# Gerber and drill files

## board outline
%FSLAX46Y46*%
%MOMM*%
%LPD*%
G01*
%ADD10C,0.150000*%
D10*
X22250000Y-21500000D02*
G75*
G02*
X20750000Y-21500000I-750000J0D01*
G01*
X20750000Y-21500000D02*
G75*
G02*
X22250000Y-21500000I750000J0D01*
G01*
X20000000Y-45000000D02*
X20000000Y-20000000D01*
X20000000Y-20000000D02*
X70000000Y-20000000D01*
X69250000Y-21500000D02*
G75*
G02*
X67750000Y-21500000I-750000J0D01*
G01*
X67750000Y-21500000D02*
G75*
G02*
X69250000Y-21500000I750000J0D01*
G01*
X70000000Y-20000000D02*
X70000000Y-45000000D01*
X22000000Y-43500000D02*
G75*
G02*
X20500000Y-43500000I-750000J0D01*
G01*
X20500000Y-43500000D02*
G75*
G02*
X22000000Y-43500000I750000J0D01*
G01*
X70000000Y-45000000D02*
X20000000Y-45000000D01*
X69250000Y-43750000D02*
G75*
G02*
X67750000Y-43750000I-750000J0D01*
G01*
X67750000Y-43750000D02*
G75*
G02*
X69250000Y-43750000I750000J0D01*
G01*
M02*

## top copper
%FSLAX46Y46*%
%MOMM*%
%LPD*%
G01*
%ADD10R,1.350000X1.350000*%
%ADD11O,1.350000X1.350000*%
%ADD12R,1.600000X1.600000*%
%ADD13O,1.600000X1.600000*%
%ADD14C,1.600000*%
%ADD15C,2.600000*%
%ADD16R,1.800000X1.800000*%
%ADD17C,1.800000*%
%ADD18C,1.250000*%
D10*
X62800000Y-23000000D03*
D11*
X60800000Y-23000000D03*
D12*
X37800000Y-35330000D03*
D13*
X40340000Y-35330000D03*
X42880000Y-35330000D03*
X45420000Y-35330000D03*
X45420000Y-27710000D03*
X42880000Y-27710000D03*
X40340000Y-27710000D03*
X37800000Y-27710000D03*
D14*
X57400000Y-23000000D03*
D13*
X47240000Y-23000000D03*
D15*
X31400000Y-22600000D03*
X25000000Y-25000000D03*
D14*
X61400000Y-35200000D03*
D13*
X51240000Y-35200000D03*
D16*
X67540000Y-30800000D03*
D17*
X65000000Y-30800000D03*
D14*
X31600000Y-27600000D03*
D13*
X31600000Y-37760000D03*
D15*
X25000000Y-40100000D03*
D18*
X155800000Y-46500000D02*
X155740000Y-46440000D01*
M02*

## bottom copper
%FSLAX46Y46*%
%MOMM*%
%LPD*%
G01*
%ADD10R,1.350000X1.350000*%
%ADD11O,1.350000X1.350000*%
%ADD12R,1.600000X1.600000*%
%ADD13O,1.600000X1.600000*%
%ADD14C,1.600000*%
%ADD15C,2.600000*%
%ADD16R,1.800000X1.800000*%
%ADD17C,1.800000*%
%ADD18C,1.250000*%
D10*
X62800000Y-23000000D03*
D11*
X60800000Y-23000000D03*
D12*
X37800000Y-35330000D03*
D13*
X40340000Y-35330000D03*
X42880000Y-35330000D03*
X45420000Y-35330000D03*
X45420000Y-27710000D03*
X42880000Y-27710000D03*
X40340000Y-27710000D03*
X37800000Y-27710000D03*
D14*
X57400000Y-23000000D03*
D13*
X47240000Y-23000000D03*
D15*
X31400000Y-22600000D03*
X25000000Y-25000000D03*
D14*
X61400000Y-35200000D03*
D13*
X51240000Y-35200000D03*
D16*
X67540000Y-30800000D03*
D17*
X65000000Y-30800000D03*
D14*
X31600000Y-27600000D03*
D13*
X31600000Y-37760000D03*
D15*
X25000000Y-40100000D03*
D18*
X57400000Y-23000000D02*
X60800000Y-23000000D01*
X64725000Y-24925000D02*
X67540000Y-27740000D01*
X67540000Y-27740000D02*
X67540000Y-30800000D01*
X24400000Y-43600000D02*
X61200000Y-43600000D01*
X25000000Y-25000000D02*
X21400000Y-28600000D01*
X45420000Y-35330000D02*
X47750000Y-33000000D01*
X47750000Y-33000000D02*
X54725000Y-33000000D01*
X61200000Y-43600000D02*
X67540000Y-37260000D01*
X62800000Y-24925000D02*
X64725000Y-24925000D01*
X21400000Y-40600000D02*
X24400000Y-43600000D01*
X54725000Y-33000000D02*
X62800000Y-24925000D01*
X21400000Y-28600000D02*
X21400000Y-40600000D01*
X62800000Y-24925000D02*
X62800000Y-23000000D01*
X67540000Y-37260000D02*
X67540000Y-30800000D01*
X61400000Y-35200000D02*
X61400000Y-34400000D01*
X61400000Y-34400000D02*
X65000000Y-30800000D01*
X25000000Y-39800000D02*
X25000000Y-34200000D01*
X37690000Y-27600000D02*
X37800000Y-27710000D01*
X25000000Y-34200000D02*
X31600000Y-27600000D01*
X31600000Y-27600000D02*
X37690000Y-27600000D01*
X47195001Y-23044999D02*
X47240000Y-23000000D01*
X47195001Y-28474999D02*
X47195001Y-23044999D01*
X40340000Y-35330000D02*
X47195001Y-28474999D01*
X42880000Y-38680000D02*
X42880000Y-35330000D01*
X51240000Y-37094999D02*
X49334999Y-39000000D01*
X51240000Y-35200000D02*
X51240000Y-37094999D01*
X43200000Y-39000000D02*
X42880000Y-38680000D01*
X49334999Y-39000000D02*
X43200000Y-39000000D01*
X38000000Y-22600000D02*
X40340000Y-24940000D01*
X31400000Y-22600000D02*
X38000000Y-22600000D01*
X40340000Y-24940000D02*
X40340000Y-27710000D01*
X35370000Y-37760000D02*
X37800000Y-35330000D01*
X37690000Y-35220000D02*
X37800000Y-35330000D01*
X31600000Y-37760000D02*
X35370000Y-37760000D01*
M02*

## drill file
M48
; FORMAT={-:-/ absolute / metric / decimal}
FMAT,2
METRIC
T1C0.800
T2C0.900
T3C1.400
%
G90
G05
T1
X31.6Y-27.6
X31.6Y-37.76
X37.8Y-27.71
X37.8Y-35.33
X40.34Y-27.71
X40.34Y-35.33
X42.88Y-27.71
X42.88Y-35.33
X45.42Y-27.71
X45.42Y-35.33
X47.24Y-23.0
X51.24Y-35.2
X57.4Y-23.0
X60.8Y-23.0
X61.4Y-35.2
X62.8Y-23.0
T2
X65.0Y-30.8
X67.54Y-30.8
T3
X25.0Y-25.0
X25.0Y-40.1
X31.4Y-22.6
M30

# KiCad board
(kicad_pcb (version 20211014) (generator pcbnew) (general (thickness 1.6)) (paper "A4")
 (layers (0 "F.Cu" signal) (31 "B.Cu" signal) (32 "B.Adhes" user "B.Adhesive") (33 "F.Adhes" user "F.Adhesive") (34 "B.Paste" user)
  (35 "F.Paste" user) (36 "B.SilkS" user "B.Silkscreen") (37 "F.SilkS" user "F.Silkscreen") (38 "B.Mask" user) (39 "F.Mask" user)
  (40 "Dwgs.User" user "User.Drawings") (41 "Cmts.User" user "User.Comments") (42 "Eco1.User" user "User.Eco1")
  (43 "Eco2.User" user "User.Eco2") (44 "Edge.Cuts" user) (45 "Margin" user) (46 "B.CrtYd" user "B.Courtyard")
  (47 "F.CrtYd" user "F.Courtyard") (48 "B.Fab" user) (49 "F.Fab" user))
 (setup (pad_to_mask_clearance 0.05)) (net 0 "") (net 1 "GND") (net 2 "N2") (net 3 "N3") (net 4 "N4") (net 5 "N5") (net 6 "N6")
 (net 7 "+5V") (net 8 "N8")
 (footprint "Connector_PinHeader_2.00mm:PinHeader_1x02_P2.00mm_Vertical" (layer "F.Cu") (at 62.8 23 -90)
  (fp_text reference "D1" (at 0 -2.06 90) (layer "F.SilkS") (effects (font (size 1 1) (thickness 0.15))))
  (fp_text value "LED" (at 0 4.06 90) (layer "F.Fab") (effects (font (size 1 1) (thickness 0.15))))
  (pad "1" thru_hole rect locked (at 0 0 270) (size 1.35 1.35) (drill 0.8) (layers *.Cu *.Mask) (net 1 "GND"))
  (pad "2" thru_hole oval locked (at 0 2 270) (size 1.35 1.35) (drill 0.8) (layers *.Cu *.Mask) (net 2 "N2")))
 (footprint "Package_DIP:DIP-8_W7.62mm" (layer "F.Cu") (at 37.8 35.33 90)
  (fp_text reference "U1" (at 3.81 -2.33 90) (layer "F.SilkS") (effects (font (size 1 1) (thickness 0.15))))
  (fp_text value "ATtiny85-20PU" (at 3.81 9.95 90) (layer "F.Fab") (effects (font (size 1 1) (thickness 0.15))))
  (pad "1" thru_hole rect locked (at 0 0 90) (size 1.6 1.6) (drill 0.8) (layers *.Cu *.Mask) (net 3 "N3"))
  (pad "2" thru_hole oval locked (at 0 2.54 90) (size 1.6 1.6) (drill 0.8) (layers *.Cu *.Mask) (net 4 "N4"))
  (pad "3" thru_hole oval locked (at 0 5.08 90) (size 1.6 1.6) (drill 0.8) (layers *.Cu *.Mask) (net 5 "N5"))
  (pad "4" thru_hole oval locked (at 0 7.62 90) (size 1.6 1.6) (drill 0.8) (layers *.Cu *.Mask) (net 1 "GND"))
  (pad "5" thru_hole oval locked (at 7.62 7.62 90) (size 1.6 1.6) (drill 0.8) (layers *.Cu *.Mask))
  (pad "6" thru_hole oval locked (at 7.62 5.08 90) (size 1.6 1.6) (drill 0.8) (layers *.Cu *.Mask))
  (pad "7" thru_hole oval locked (at 7.62 2.54 90) (size 1.6 1.6) (drill 0.8) (layers *.Cu *.Mask) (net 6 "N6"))
  (pad "8" thru_hole oval locked (at 7.62 0 90) (size 1.6 1.6) (drill 0.8) (layers *.Cu *.Mask) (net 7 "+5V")))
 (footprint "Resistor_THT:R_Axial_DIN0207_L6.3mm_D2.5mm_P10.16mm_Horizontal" (layer "F.Cu") (at 57.4 23 180)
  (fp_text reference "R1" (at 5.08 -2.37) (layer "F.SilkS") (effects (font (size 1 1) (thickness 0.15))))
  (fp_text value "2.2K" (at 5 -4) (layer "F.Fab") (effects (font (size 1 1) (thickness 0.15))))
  (pad "1" thru_hole circle locked (at 0 0 180) (size 1.6 1.6) (drill 0.8) (layers *.Cu *.Mask) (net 2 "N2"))
  (pad "2" thru_hole oval locked (at 10.16 0 180) (size 1.6 1.6) (drill 0.8) (layers *.Cu *.Mask) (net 4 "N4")))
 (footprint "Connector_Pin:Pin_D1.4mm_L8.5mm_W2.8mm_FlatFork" (layer "F.Cu") (at 31.4 22.6)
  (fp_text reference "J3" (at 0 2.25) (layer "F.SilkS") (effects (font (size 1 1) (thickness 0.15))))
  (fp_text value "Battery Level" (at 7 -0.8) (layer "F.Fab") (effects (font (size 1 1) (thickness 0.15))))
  (pad "1" thru_hole circle locked (at 0 0) (size 2.6 2.6) (drill 1.4) (layers *.Cu *.Mask) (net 6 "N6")))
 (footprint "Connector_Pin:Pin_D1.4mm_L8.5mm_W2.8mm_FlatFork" (layer "F.Cu") (at 25 25)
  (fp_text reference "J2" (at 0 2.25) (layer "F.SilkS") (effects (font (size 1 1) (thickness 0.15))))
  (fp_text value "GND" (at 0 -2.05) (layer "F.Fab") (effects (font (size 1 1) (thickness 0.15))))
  (pad "1" thru_hole circle locked (at 0 0) (size 2.6 2.6) (drill 1.4) (layers *.Cu *.Mask) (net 1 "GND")))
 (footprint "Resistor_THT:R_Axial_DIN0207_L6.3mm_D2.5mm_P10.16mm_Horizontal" (layer "F.Cu") (at 61.4 35.2 180)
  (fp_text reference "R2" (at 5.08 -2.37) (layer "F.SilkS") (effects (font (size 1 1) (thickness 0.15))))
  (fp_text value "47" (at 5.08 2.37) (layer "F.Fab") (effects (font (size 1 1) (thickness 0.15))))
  (pad "1" thru_hole circle locked (at 0 0 180) (size 1.6 1.6) (drill 0.8) (layers *.Cu *.Mask) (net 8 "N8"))
  (pad "2" thru_hole oval locked (at 10.16 0 180) (size 1.6 1.6) (drill 0.8) (layers *.Cu *.Mask) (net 5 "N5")))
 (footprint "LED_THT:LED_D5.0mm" (layer "F.Cu") (at 67.54 30.8 180)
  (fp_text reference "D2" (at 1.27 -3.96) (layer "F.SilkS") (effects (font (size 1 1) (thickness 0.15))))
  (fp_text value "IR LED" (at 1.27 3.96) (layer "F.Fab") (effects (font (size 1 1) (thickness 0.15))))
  (pad "1" thru_hole rect locked (at 0 0 180) (size 1.8 1.8) (drill 0.9) (layers *.Cu *.Mask) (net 1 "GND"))
  (pad "2" thru_hole circle locked (at 2.54 0 180) (size 1.8 1.8) (drill 0.9) (layers *.Cu *.Mask) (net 8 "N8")))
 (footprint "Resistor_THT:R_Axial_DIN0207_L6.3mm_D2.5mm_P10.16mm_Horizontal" (layer "F.Cu") (at 31.6 27.6 -90)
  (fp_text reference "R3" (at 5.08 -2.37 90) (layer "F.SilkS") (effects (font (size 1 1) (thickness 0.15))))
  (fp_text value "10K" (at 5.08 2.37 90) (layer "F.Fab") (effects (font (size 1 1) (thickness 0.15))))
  (pad "1" thru_hole circle locked (at 0 0 270) (size 1.6 1.6) (drill 0.8) (layers *.Cu *.Mask) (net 7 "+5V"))
  (pad "2" thru_hole oval locked (at 10.16 0 270) (size 1.6 1.6) (drill 0.8) (layers *.Cu *.Mask) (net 3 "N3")))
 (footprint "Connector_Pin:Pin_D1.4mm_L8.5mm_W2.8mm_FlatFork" (layer "F.Cu") (at 25 40.1)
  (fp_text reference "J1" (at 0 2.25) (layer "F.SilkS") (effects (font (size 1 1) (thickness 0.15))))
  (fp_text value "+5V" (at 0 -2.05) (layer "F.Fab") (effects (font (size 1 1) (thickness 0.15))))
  (pad "1" thru_hole circle locked (at 0 0) (size 2.6 2.6) (drill 1.4) (layers *.Cu *.Mask) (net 7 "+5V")))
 (gr_circle (center 21.5 21.5) (end 22.25 21.5) (layer "Edge.Cuts") (width 0.15) (fill none))
 (gr_line (start 20 45) (end 20 20) (layer "Edge.Cuts") (width 0.15))
 (gr_line (start 20 20) (end 70 20) (layer "Edge.Cuts") (width 0.15))
 (gr_circle (center 68.5 21.5) (end 69.25 21.5) (layer "Edge.Cuts") (width 0.15) (fill none))
 (gr_line (start 70 20) (end 70 45) (layer "Edge.Cuts") (width 0.15))
 (gr_circle (center 21.25 43.5) (end 22 43.5) (layer "Edge.Cuts") (width 0.15) (fill none))
 (gr_line (start 70 45) (end 20 45) (layer "Edge.Cuts") (width 0.15))
 (gr_circle (center 68.5 43.75) (end 69.25 43.75) (layer "Edge.Cuts") (width 0.15) (fill none))
 (segment (start 57.4 23) (end 60.8 23) (width 1.25) (layer "B.Cu") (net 2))
 (segment (start 155.8 46.5) (end 155.74 46.44) (width 1.25) (layer "F.Cu") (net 1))
 (segment (start 64.725 24.925) (end 67.54 27.74) (width 1.25) (layer "B.Cu") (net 1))
 (segment (start 67.54 27.74) (end 67.54 30.8) (width 1.25) (layer "B.Cu") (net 1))
 (segment (start 24.4 43.6) (end 61.2 43.6) (width 1.25) (layer "B.Cu") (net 1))
 (segment (start 25 25) (end 21.4 28.6) (width 1.25) (layer "B.Cu") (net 1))
 (segment (start 45.42 35.33) (end 47.75 33) (width 1.25) (layer "B.Cu") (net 1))
 (segment (start 47.75 33) (end 54.725 33) (width 1.25) (layer "B.Cu") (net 1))
 (segment (start 61.2 43.6) (end 67.54 37.26) (width 1.25) (layer "B.Cu") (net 1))
 (segment (start 62.8 24.925) (end 64.725 24.925) (width 1.25) (layer "B.Cu") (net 1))
 (segment (start 21.4 40.6) (end 24.4 43.6) (width 1.25) (layer "B.Cu") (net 1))
 (segment (start 54.725 33) (end 62.8 24.925) (width 1.25) (layer "B.Cu") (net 1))
 (segment (start 21.4 28.6) (end 21.4 40.6) (width 1.25) (layer "B.Cu") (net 1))
 (segment (start 62.8 24.925) (end 62.8 23) (width 1.25) (layer "B.Cu") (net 1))
 (segment (start 67.54 37.26) (end 67.54 30.8) (width 1.25) (layer "B.Cu") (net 1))
 (segment (start 61.4 35.2) (end 61.4 34.4) (width 1.25) (layer "B.Cu") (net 8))
 (segment (start 61.4 34.4) (end 65 30.8) (width 1.25) (layer "B.Cu") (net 8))
 (segment (start 25 39.8) (end 25 34.2) (width 1.25) (layer "B.Cu") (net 7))
 (segment (start 37.69 27.6) (end 37.8 27.71) (width 1.25) (layer "B.Cu") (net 7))
 (segment (start 25 34.2) (end 31.6 27.6) (width 1.25) (layer "B.Cu") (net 7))
 (segment (start 31.6 27.6) (end 37.69 27.6) (width 1.25) (layer "B.Cu") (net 7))
 (segment (start 47.195001 23.044999) (end 47.24 23) (width 1.25) (layer "B.Cu") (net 4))
 (segment (start 47.195001 28.474999) (end 47.195001 23.044999) (width 1.25) (layer "B.Cu") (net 4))
 (segment (start 40.34 35.33) (end 47.195001 28.474999) (width 1.25) (layer "B.Cu") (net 4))
 (segment (start 42.88 38.68) (end 42.88 35.33) (width 1.25) (layer "B.Cu") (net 5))
 (segment (start 51.24 37.094999) (end 49.334999 39) (width 1.25) (layer "B.Cu") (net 5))
 (segment (start 51.24 35.2) (end 51.24 37.094999) (width 1.25) (layer "B.Cu") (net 5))
 (segment (start 43.2 39) (end 42.88 38.68) (width 1.25) (layer "B.Cu") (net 5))
 (segment (start 49.334999 39) (end 43.2 39) (width 1.25) (layer "B.Cu") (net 5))
 (segment (start 38 22.6) (end 40.34 24.94) (width 1.25) (layer "B.Cu") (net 6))
 (segment (start 31.4 22.6) (end 38 22.6) (width 1.25) (layer "B.Cu") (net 6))
 (segment (start 40.34 24.94) (end 40.34 27.71) (width 1.25) (layer "B.Cu") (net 6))
 (segment (start 35.37 37.76) (end 37.8 35.33) (width 1.25) (layer "B.Cu") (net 3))
 (segment (start 37.69 35.22) (end 37.8 35.33) (width 1.25) (layer "B.Cu") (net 3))
 (segment (start 31.6 37.76) (end 35.37 37.76) (width 1.25) (layer "B.Cu") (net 3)))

